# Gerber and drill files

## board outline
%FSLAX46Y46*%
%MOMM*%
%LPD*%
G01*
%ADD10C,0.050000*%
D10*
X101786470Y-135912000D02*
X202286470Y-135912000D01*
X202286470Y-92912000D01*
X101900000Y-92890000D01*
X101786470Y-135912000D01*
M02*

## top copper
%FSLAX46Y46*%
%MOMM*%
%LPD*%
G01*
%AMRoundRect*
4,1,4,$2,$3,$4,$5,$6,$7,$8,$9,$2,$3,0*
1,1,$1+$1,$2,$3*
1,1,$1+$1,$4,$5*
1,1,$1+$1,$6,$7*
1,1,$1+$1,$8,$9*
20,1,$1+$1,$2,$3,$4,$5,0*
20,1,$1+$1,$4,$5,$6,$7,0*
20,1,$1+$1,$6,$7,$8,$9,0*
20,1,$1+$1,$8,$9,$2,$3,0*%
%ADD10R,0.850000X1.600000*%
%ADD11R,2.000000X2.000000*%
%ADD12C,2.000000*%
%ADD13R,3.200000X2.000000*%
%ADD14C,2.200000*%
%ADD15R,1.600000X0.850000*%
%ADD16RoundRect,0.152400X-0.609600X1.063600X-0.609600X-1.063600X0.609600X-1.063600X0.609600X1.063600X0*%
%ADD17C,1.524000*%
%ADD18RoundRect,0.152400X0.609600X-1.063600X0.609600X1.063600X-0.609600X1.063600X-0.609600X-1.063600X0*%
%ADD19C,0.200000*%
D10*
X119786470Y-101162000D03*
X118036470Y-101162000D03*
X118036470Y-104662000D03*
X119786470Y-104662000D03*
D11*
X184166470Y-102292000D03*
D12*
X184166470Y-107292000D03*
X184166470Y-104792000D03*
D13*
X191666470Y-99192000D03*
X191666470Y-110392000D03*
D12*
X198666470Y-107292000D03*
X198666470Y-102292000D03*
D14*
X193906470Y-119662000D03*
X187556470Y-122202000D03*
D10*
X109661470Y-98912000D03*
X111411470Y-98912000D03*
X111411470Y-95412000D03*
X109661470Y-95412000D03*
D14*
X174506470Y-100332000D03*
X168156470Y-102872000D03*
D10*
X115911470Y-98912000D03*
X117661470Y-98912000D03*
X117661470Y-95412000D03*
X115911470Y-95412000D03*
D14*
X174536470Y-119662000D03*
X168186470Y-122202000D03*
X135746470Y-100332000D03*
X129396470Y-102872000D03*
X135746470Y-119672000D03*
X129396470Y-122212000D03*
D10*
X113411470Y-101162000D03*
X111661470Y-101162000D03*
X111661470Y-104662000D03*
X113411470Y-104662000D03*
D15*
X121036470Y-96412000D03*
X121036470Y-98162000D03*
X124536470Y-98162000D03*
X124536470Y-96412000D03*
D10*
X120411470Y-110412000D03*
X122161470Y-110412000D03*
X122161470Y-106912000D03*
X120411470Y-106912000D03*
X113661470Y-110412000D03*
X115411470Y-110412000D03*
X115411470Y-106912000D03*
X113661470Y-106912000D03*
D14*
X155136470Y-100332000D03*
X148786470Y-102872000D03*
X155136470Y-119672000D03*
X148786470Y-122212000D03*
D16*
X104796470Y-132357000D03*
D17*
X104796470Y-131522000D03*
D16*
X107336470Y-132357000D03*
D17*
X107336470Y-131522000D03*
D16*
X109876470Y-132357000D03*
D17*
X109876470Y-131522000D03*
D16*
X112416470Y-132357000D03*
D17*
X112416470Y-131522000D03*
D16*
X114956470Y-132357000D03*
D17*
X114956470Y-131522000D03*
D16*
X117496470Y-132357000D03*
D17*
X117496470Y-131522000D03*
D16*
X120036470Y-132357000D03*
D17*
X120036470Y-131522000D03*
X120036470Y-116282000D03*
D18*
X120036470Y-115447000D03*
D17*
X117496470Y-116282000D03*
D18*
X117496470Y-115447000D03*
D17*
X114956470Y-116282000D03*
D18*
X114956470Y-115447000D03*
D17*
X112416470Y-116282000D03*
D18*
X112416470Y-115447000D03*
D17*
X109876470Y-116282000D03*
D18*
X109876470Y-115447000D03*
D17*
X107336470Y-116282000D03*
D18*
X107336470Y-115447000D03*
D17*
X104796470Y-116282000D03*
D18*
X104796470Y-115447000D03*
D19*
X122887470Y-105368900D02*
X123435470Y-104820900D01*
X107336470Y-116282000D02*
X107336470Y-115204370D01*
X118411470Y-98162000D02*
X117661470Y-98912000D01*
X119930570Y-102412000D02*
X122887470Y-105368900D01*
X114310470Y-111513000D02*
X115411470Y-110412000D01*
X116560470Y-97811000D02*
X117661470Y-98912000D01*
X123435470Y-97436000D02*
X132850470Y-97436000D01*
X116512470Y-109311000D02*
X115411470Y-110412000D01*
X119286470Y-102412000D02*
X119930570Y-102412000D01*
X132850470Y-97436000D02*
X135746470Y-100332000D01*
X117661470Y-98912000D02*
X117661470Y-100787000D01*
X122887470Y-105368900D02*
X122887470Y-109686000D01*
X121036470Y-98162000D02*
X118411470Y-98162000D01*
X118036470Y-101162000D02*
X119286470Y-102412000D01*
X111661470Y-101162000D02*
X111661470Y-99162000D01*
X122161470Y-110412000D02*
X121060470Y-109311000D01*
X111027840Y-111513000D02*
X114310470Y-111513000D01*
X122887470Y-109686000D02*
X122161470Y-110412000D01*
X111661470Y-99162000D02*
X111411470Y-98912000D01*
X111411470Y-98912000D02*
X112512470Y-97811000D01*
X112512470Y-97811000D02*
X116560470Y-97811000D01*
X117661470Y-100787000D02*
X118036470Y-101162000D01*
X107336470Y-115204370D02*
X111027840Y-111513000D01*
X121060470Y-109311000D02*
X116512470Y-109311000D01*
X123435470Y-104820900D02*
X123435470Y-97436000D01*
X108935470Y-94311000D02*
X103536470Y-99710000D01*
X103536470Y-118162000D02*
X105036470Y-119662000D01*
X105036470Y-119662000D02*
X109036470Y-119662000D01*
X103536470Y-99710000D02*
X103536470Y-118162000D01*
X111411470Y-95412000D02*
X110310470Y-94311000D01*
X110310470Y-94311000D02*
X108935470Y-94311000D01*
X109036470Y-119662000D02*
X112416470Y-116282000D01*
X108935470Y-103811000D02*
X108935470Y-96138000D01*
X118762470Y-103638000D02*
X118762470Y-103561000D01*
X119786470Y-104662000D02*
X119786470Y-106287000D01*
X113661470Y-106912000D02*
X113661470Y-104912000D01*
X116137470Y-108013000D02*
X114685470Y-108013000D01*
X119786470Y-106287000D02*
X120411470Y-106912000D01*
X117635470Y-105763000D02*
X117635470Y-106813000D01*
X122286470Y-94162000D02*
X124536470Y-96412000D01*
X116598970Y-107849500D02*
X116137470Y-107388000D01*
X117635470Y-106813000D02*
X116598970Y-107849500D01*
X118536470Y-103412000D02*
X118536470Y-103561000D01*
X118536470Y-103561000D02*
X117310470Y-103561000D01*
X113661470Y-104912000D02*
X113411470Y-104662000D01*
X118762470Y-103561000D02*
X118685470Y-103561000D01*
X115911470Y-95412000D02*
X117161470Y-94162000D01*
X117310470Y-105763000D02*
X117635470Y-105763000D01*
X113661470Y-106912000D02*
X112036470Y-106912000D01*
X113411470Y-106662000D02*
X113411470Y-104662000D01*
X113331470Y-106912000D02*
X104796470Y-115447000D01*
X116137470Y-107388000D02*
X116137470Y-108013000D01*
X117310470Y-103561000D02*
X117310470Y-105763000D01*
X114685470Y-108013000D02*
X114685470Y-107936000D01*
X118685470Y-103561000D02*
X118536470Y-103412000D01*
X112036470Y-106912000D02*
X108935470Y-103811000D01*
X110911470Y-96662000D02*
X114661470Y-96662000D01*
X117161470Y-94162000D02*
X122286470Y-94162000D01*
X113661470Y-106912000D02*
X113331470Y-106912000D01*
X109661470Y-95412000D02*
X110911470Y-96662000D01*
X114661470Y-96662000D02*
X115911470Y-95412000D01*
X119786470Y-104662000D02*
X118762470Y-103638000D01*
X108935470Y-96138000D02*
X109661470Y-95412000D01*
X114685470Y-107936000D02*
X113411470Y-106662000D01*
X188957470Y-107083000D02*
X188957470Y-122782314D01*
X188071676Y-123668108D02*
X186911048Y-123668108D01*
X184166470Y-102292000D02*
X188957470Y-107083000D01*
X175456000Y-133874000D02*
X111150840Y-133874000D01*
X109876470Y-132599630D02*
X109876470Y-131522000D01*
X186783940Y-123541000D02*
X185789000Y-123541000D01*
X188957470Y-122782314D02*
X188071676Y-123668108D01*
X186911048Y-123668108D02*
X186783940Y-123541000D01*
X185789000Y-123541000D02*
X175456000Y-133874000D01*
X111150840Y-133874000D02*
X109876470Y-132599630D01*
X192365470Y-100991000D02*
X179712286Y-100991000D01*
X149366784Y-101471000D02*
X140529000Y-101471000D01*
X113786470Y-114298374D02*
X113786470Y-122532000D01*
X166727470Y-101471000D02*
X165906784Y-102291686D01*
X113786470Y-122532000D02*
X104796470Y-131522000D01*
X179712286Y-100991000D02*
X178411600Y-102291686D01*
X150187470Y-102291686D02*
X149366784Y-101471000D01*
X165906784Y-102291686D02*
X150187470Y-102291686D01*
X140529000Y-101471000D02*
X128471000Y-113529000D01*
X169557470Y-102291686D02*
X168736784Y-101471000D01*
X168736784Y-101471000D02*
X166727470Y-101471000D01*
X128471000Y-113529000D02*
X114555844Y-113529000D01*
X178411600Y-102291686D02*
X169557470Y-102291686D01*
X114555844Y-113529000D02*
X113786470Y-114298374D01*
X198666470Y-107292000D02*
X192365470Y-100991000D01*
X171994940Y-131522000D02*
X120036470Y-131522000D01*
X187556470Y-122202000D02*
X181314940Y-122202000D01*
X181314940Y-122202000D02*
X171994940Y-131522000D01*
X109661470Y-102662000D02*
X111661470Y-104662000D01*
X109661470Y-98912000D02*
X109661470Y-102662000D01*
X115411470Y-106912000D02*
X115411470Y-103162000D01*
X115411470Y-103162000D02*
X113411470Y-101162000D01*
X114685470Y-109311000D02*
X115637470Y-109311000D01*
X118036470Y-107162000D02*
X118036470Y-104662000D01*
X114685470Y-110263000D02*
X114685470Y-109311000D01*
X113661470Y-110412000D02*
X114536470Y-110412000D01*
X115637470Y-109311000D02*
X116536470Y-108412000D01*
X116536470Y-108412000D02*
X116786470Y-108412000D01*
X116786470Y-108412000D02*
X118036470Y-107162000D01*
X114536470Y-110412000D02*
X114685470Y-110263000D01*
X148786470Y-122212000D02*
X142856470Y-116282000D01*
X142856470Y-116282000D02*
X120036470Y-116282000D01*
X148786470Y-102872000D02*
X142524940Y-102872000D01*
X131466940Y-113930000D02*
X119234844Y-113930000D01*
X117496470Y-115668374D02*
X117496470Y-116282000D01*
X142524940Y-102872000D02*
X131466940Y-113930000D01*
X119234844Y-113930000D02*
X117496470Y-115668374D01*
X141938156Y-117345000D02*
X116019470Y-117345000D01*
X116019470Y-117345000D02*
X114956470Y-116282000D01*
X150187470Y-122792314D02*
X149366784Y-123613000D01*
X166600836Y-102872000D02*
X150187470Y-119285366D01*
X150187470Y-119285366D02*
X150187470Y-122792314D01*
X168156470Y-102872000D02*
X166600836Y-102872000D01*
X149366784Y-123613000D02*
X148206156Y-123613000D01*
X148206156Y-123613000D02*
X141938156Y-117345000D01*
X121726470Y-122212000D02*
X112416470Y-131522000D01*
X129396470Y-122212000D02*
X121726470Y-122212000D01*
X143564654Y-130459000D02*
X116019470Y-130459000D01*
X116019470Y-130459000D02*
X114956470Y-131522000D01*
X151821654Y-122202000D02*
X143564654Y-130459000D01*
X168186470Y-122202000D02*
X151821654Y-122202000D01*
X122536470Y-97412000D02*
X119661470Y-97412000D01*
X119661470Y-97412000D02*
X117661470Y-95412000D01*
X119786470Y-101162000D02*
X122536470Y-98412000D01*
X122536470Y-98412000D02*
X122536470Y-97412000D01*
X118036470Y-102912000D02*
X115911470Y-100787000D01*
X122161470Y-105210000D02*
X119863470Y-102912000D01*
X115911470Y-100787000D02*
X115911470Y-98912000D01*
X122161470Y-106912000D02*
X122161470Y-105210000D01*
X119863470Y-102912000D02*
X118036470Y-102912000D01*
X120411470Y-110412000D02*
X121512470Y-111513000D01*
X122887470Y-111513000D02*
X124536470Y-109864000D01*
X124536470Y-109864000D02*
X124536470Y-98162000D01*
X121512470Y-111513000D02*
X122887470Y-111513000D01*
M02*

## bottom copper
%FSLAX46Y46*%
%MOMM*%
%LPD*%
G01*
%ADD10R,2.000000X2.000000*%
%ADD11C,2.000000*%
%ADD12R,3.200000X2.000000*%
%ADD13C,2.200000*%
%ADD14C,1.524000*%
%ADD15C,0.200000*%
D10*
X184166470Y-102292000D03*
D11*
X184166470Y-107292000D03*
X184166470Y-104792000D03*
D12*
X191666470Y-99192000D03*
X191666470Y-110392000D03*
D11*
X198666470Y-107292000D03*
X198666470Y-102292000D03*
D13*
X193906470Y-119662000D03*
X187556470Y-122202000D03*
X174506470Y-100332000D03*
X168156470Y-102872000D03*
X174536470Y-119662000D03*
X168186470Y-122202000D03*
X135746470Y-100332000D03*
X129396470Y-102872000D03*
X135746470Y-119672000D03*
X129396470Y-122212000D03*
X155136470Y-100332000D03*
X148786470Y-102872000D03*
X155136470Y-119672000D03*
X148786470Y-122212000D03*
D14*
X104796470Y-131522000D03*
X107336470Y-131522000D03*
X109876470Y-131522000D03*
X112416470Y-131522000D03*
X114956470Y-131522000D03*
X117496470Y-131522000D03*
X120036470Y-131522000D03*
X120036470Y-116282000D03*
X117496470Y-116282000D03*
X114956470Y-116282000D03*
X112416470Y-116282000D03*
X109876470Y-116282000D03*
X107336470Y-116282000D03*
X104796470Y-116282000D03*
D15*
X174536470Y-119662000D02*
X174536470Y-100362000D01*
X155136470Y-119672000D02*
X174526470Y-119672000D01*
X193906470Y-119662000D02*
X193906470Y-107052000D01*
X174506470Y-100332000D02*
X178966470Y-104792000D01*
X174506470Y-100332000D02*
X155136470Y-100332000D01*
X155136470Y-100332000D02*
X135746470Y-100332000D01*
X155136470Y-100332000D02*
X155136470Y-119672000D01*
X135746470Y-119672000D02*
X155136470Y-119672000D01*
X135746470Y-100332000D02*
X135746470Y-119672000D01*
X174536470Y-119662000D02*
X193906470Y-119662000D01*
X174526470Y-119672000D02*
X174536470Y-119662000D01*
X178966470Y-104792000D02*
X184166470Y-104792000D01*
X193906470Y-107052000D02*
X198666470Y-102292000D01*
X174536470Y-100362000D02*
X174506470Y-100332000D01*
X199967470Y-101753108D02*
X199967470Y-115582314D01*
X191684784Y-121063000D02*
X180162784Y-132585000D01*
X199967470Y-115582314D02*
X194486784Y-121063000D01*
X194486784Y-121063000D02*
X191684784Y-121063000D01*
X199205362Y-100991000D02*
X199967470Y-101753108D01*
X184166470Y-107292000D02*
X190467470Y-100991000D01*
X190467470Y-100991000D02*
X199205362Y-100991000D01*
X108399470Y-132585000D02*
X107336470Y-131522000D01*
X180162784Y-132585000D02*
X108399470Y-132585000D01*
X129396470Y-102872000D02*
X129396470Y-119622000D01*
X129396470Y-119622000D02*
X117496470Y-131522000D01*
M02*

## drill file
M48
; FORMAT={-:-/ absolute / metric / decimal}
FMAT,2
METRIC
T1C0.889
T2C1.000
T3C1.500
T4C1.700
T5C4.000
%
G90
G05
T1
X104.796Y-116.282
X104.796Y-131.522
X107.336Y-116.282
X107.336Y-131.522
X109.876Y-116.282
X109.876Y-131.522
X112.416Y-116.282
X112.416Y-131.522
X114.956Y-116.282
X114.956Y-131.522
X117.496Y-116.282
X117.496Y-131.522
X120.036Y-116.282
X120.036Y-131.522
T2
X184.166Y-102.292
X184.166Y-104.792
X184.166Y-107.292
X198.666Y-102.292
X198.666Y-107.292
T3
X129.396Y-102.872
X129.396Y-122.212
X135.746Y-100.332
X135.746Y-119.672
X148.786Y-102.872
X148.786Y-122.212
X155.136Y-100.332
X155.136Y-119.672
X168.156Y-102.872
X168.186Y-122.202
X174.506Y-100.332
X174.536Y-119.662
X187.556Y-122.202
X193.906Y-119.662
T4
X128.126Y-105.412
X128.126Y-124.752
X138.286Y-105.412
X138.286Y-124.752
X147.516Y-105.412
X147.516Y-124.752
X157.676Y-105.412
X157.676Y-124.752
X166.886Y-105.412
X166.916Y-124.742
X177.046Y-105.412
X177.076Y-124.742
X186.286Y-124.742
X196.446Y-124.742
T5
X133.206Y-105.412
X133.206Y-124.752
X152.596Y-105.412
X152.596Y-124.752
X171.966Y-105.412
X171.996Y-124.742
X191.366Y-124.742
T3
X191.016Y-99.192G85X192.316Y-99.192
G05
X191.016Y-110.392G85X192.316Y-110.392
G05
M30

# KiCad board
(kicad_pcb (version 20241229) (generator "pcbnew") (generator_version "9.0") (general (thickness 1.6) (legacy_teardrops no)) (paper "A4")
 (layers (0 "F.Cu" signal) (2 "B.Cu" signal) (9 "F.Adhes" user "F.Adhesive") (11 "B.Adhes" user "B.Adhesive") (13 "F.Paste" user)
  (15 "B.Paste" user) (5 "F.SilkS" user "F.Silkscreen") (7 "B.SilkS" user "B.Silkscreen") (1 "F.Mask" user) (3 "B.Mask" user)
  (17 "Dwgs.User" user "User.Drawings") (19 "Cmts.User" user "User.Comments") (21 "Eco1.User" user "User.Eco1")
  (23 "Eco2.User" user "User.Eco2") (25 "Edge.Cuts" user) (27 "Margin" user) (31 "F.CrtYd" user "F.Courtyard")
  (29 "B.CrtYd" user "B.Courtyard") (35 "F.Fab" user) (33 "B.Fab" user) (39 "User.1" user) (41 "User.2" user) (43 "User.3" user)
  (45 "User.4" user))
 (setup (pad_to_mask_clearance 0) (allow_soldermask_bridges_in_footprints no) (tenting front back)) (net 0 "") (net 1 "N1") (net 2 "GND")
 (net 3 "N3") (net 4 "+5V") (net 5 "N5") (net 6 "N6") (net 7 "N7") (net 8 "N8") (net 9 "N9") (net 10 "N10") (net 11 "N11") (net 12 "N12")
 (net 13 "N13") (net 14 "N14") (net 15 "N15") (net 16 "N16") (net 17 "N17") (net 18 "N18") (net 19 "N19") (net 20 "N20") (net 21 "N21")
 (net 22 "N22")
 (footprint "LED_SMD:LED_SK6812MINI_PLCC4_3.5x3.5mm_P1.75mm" (layer "F.Cu") (at 118.91147 102.912 -90)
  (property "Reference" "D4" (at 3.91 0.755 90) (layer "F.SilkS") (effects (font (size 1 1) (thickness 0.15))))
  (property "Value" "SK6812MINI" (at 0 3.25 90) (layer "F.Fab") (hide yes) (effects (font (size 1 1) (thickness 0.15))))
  (pad "1" smd rect (at -1.75 -0.875 270) (size 1.6 0.85) (layers "F.Cu" "F.Mask" "F.Paste") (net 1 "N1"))
  (pad "2" smd rect (at -1.75 0.875 270) (size 1.6 0.85) (layers "F.Cu" "F.Mask" "F.Paste") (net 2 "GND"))
  (pad "3" smd rect (at 1.75 0.875 270) (size 1.6 0.85) (layers "F.Cu" "F.Mask" "F.Paste") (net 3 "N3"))
  (pad "4" smd rect (at 1.75 -0.875 270) (size 1.6 0.85) (layers "F.Cu" "F.Mask" "F.Paste") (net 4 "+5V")))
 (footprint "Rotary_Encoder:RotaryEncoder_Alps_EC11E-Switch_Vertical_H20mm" (layer "F.Cu") (at 184.16647 102.292)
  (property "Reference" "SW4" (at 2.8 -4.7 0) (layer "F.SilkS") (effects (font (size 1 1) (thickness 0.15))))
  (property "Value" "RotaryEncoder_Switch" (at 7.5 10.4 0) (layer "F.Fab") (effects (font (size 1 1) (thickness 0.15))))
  (pad "A" thru_hole rect (at 0 0) (size 2 2) (drill 1) (layers "*.Cu" "*.Mask") (remove_unused_layers no) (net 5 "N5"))
  (pad "B" thru_hole circle (at 0 5) (size 2 2) (drill 1) (layers "*.Cu" "*.Mask") (remove_unused_layers no) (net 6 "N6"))
  (pad "C" thru_hole circle (at 0 2.5) (size 2 2) (drill 1) (layers "*.Cu" "*.Mask") (remove_unused_layers no) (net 2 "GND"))
  (pad "MP" thru_hole rect (at 7.5 -3.1) (size 3.2 2) (drill oval 2.8 1.5) (layers "*.Cu" "*.Mask") (remove_unused_layers no))
  (pad "MP" thru_hole rect (at 7.5 8.1) (size 3.2 2) (drill oval 2.8 1.5) (layers "*.Cu" "*.Mask") (remove_unused_layers no))
  (pad "S1" thru_hole circle (at 14.5 5) (size 2 2) (drill 1) (layers "*.Cu" "*.Mask") (remove_unused_layers no) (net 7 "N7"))
  (pad "S2" thru_hole circle (at 14.5 0) (size 2 2) (drill 1) (layers "*.Cu" "*.Mask") (remove_unused_layers no) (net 2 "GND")))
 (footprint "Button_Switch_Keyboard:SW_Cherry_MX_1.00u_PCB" (layer "F.Cu") (at 193.90647 119.662)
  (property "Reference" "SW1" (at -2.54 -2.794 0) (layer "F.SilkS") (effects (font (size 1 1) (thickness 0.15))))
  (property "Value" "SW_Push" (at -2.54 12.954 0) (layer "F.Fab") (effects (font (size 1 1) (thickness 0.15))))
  (pad "" np_thru_hole circle (at -7.62 5.08) (size 1.7 1.7) (drill 1.7) (layers "*.Cu" "*.Mask"))
  (pad "" np_thru_hole circle (at -2.54 5.08) (size 4 4) (drill 4) (layers "*.Cu" "*.Mask"))
  (pad "" np_thru_hole circle (at 2.54 5.08) (size 1.7 1.7) (drill 1.7) (layers "*.Cu" "*.Mask"))
  (pad "1" thru_hole circle (at 0 0) (size 2.2 2.2) (drill 1.5) (layers "*.Cu" "*.Mask") (remove_unused_layers no) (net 2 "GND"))
  (pad "2" thru_hole circle (at -6.35 2.54) (size 2.2 2.2) (drill 1.5) (layers "*.Cu" "*.Mask") (remove_unused_layers no) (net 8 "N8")))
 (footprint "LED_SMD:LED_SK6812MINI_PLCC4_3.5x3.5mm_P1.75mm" (layer "F.Cu") (at 110.53647 97.162 90)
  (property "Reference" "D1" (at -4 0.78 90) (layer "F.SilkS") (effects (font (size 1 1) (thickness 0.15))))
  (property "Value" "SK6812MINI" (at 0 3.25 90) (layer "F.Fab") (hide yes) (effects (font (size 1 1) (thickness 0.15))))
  (pad "1" smd rect (at -1.75 -0.875 90) (size 1.6 0.85) (layers "F.Cu" "F.Mask" "F.Paste") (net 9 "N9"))
  (pad "2" smd rect (at -1.75 0.875 90) (size 1.6 0.85) (layers "F.Cu" "F.Mask" "F.Paste") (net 2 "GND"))
  (pad "3" smd rect (at 1.75 0.875 90) (size 1.6 0.85) (layers "F.Cu" "F.Mask" "F.Paste") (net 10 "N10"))
  (pad "4" smd rect (at 1.75 -0.875 90) (size 1.6 0.85) (layers "F.Cu" "F.Mask" "F.Paste") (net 4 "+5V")))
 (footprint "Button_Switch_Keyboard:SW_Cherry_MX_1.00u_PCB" (layer "F.Cu") (at 174.50647 100.332)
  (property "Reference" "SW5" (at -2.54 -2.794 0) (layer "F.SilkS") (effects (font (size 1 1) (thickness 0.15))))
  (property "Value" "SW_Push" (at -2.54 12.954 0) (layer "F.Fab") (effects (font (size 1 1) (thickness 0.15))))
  (pad "" np_thru_hole circle (at -7.62 5.08) (size 1.7 1.7) (drill 1.7) (layers "*.Cu" "*.Mask"))
  (pad "" np_thru_hole circle (at -2.54 5.08) (size 4 4) (drill 4) (layers "*.Cu" "*.Mask"))
  (pad "" np_thru_hole circle (at 2.54 5.08) (size 1.7 1.7) (drill 1.7) (layers "*.Cu" "*.Mask"))
  (pad "1" thru_hole circle (at 0 0) (size 2.2 2.2) (drill 1.5) (layers "*.Cu" "*.Mask") (remove_unused_layers no) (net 2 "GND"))
  (pad "2" thru_hole circle (at -6.35 2.54) (size 2.2 2.2) (drill 1.5) (layers "*.Cu" "*.Mask") (remove_unused_layers no) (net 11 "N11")))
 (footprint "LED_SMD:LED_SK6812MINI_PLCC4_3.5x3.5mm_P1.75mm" (layer "F.Cu") (at 116.78647 97.162 90)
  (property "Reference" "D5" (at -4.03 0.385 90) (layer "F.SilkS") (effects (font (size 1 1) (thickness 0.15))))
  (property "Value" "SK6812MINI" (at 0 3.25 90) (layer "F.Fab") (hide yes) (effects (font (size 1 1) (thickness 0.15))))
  (pad "1" smd rect (at -1.75 -0.875 90) (size 1.6 0.85) (layers "F.Cu" "F.Mask" "F.Paste") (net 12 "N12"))
  (pad "2" smd rect (at -1.75 0.875 90) (size 1.6 0.85) (layers "F.Cu" "F.Mask" "F.Paste") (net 2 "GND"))
  (pad "3" smd rect (at 1.75 0.875 90) (size 1.6 0.85) (layers "F.Cu" "F.Mask" "F.Paste") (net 1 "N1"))
  (pad "4" smd rect (at 1.75 -0.875 90) (size 1.6 0.85) (layers "F.Cu" "F.Mask" "F.Paste") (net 4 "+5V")))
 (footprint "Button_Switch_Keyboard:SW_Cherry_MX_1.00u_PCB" (layer "F.Cu") (at 174.53647 119.662)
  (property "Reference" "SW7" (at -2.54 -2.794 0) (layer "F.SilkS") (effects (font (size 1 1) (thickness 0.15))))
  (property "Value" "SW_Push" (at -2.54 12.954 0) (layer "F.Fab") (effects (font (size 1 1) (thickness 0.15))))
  (pad "" np_thru_hole circle (at -7.62 5.08) (size 1.7 1.7) (drill 1.7) (layers "*.Cu" "*.Mask"))
  (pad "" np_thru_hole circle (at -2.54 5.08) (size 4 4) (drill 4) (layers "*.Cu" "*.Mask"))
  (pad "" np_thru_hole circle (at 2.54 5.08) (size 1.7 1.7) (drill 1.7) (layers "*.Cu" "*.Mask"))
  (pad "1" thru_hole circle (at 0 0) (size 2.2 2.2) (drill 1.5) (layers "*.Cu" "*.Mask") (remove_unused_layers no) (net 2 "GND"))
  (pad "2" thru_hole circle (at -6.35 2.54) (size 2.2 2.2) (drill 1.5) (layers "*.Cu" "*.Mask") (remove_unused_layers no) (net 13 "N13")))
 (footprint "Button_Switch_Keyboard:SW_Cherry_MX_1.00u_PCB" (layer "F.Cu") (at 135.74647 100.332)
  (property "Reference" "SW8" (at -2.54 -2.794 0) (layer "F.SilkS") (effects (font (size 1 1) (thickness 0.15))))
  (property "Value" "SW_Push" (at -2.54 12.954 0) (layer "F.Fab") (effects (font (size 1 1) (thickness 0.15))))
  (pad "" np_thru_hole circle (at -7.62 5.08) (size 1.7 1.7) (drill 1.7) (layers "*.Cu" "*.Mask"))
  (pad "" np_thru_hole circle (at -2.54 5.08) (size 4 4) (drill 4) (layers "*.Cu" "*.Mask"))
  (pad "" np_thru_hole circle (at 2.54 5.08) (size 1.7 1.7) (drill 1.7) (layers "*.Cu" "*.Mask"))
  (pad "1" thru_hole circle (at 0 0) (size 2.2 2.2) (drill 1.5) (layers "*.Cu" "*.Mask") (remove_unused_layers no) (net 2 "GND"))
  (pad "2" thru_hole circle (at -6.35 2.54) (size 2.2 2.2) (drill 1.5) (layers "*.Cu" "*.Mask") (remove_unused_layers no) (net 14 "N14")))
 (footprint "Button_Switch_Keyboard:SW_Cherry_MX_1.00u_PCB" (layer "F.Cu") (at 135.74647 119.672)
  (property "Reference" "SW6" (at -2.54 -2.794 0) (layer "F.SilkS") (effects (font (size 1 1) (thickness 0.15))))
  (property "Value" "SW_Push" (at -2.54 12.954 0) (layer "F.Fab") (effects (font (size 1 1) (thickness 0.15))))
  (pad "" np_thru_hole circle (at -7.62 5.08) (size 1.7 1.7) (drill 1.7) (layers "*.Cu" "*.Mask"))
  (pad "" np_thru_hole circle (at -2.54 5.08) (size 4 4) (drill 4) (layers "*.Cu" "*.Mask"))
  (pad "" np_thru_hole circle (at 2.54 5.08) (size 1.7 1.7) (drill 1.7) (layers "*.Cu" "*.Mask"))
  (pad "1" thru_hole circle (at 0 0) (size 2.2 2.2) (drill 1.5) (layers "*.Cu" "*.Mask") (remove_unused_layers no) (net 2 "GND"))
  (pad "2" thru_hole circle (at -6.35 2.54) (size 2.2 2.2) (drill 1.5) (layers "*.Cu" "*.Mask") (remove_unused_layers no) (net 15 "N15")))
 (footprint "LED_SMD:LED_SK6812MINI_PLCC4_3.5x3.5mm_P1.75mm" (layer "F.Cu") (at 112.53647 102.912 -90)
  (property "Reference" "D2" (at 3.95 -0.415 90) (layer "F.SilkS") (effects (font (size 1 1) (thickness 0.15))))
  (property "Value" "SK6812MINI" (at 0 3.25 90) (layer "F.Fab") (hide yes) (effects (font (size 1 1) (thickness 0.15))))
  (pad "1" smd rect (at -1.75 -0.875 270) (size 1.6 0.85) (layers "F.Cu" "F.Mask" "F.Paste") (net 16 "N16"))
  (pad "2" smd rect (at -1.75 0.875 270) (size 1.6 0.85) (layers "F.Cu" "F.Mask" "F.Paste") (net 2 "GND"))
  (pad "3" smd rect (at 1.75 0.875 270) (size 1.6 0.85) (layers "F.Cu" "F.Mask" "F.Paste") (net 9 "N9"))
  (pad "4" smd rect (at 1.75 -0.875 270) (size 1.6 0.85) (layers "F.Cu" "F.Mask" "F.Paste") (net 4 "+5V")))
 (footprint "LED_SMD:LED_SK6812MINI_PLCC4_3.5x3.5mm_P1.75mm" (layer "F.Cu") (at 122.78647 97.287)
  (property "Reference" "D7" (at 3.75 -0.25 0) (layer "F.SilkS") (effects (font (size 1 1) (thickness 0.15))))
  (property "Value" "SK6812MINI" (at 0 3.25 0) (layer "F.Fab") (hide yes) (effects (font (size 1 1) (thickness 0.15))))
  (pad "1" smd rect (at -1.75 -0.875) (size 1.6 0.85) (layers "F.Cu" "F.Mask" "F.Paste") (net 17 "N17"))
  (pad "2" smd rect (at -1.75 0.875) (size 1.6 0.85) (layers "F.Cu" "F.Mask" "F.Paste") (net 2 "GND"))
  (pad "3" smd rect (at 1.75 0.875) (size 1.6 0.85) (layers "F.Cu" "F.Mask" "F.Paste") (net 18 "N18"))
  (pad "4" smd rect (at 1.75 -0.875) (size 1.6 0.85) (layers "F.Cu" "F.Mask" "F.Paste") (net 4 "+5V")))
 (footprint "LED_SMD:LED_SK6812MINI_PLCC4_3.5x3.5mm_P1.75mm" (layer "F.Cu") (at 121.28647 108.662 90)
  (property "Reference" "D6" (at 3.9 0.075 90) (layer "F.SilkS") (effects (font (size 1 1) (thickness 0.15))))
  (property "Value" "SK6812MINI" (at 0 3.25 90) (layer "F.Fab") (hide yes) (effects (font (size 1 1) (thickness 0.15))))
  (pad "1" smd rect (at -1.75 -0.875 90) (size 1.6 0.85) (layers "F.Cu" "F.Mask" "F.Paste") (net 18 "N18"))
  (pad "2" smd rect (at -1.75 0.875 90) (size 1.6 0.85) (layers "F.Cu" "F.Mask" "F.Paste") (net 2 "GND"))
  (pad "3" smd rect (at 1.75 0.875 90) (size 1.6 0.85) (layers "F.Cu" "F.Mask" "F.Paste") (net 12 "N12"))
  (pad "4" smd rect (at 1.75 -0.875 90) (size 1.6 0.85) (layers "F.Cu" "F.Mask" "F.Paste") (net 4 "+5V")))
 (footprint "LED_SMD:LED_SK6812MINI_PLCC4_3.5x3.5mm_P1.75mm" (layer "F.Cu") (at 114.53647 108.662 90)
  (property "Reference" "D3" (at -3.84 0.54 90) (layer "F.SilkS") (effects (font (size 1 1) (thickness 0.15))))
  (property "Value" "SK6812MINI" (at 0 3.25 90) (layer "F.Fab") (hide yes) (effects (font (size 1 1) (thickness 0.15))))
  (pad "1" smd rect (at -1.75 -0.875 90) (size 1.6 0.85) (layers "F.Cu" "F.Mask" "F.Paste") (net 3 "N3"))
  (pad "2" smd rect (at -1.75 0.875 90) (size 1.6 0.85) (layers "F.Cu" "F.Mask" "F.Paste") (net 2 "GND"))
  (pad "3" smd rect (at 1.75 0.875 90) (size 1.6 0.85) (layers "F.Cu" "F.Mask" "F.Paste") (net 16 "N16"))
  (pad "4" smd rect (at 1.75 -0.875 90) (size 1.6 0.85) (layers "F.Cu" "F.Mask" "F.Paste") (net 4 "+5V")))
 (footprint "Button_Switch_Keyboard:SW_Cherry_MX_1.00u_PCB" (layer "F.Cu") (at 155.13647 100.332)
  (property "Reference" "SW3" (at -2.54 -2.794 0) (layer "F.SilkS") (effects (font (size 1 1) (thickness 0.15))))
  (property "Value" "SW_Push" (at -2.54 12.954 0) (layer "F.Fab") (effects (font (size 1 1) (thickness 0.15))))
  (pad "" np_thru_hole circle (at -7.62 5.08) (size 1.7 1.7) (drill 1.7) (layers "*.Cu" "*.Mask"))
  (pad "" np_thru_hole circle (at -2.54 5.08) (size 4 4) (drill 4) (layers "*.Cu" "*.Mask"))
  (pad "" np_thru_hole circle (at 2.54 5.08) (size 1.7 1.7) (drill 1.7) (layers "*.Cu" "*.Mask"))
  (pad "1" thru_hole circle (at 0 0) (size 2.2 2.2) (drill 1.5) (layers "*.Cu" "*.Mask") (remove_unused_layers no) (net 2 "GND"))
  (pad "2" thru_hole circle (at -6.35 2.54) (size 2.2 2.2) (drill 1.5) (layers "*.Cu" "*.Mask") (remove_unused_layers no) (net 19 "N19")))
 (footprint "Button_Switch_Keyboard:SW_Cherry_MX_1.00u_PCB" (layer "F.Cu") (at 155.13647 119.672)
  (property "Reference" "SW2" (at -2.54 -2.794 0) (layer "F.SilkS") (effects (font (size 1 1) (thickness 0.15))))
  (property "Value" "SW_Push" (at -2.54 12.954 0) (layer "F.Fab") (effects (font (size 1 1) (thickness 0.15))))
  (pad "" np_thru_hole circle (at -7.62 5.08) (size 1.7 1.7) (drill 1.7) (layers "*.Cu" "*.Mask"))
  (pad "" np_thru_hole circle (at -2.54 5.08) (size 4 4) (drill 4) (layers "*.Cu" "*.Mask"))
  (pad "" np_thru_hole circle (at 2.54 5.08) (size 1.7 1.7) (drill 1.7) (layers "*.Cu" "*.Mask"))
  (pad "1" thru_hole circle (at 0 0) (size 2.2 2.2) (drill 1.5) (layers "*.Cu" "*.Mask") (remove_unused_layers no) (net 2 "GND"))
  (pad "2" thru_hole circle (at -6.35 2.54) (size 2.2 2.2) (drill 1.5) (layers "*.Cu" "*.Mask") (remove_unused_layers no) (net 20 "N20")))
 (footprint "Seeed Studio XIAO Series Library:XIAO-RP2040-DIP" (layer "F.Cu") (at 112.41647 123.902 90)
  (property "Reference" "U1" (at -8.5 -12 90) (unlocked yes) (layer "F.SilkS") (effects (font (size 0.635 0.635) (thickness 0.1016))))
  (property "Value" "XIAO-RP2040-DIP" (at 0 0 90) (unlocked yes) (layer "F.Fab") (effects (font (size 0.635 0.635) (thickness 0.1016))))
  (pad "1" smd roundrect (at -8.455 -7.62 270) (size 2.432 1.524) (layers "F.Cu" "F.Mask") (roundrect_rratio 0.1) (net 7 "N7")
   (thermal_bridge_angle 45))
  (pad "1" thru_hole circle (at -7.62 -7.62 270) (size 1.524 1.524) (drill 0.889) (layers "*.Cu" "*.Mask") (remove_unused_layers no)
   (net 7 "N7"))
  (pad "2" smd roundrect (at -8.455 -5.08 270) (size 2.432 1.524) (layers "F.Cu" "F.Mask") (roundrect_rratio 0.1) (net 6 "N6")
   (thermal_bridge_angle 45))
  (pad "2" thru_hole circle (at -7.62 -5.08 270) (size 1.524 1.524) (drill 0.889) (layers "*.Cu" "*.Mask") (remove_unused_layers no)
   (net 6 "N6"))
  (pad "3" smd roundrect (at -8.455 -2.54 270) (size 2.432 1.524) (layers "F.Cu" "F.Mask") (roundrect_rratio 0.1) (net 5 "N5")
   (thermal_bridge_angle 45))
  (pad "3" thru_hole circle (at -7.62 -2.54 270) (size 1.524 1.524) (drill 0.889) (layers "*.Cu" "*.Mask") (remove_unused_layers no)
   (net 5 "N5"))
  (pad "4" smd roundrect (at -8.455 0 270) (size 2.432 1.524) (layers "F.Cu" "F.Mask") (roundrect_rratio 0.1) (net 15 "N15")
   (thermal_bridge_angle 45))
  (pad "4" thru_hole circle (at -7.62 0 270) (size 1.524 1.524) (drill 0.889) (layers "*.Cu" "*.Mask") (remove_unused_layers no)
   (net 15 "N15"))
  (pad "5" smd roundrect (at -8.455 2.54 270) (size 2.432 1.524) (layers "F.Cu" "F.Mask") (roundrect_rratio 0.1) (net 13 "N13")
   (thermal_bridge_angle 45))
  (pad "5" thru_hole circle (at -7.62 2.54 270) (size 1.524 1.524) (drill 0.889) (layers "*.Cu" "*.Mask") (remove_unused_layers no)
   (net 13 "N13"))
  (pad "6" smd roundrect (at -8.455 5.08 270) (size 2.432 1.524) (layers "F.Cu" "F.Mask") (roundrect_rratio 0.1) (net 14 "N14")
   (thermal_bridge_angle 45))
  (pad "6" thru_hole circle (at -7.62 5.08 270) (size 1.524 1.524) (drill 0.889) (layers "*.Cu" "*.Mask") (remove_unused_layers no)
   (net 14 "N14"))
  (pad "7" smd roundrect (at -8.455 7.62 270) (size 2.432 1.524) (layers "F.Cu" "F.Mask") (roundrect_rratio 0.1) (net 8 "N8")
   (thermal_bridge_angle 45))
  (pad "7" thru_hole circle (at -7.62 7.62 270) (size 1.524 1.524) (drill 0.889) (layers "*.Cu" "*.Mask") (remove_unused_layers no)
   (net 8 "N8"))
  (pad "8" thru_hole circle (at 7.62 7.62 90) (size 1.524 1.524) (drill 0.889) (layers "*.Cu" "*.Mask") (remove_unused_layers no)
   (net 20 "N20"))
  (pad "8" smd roundrect (at 8.455 7.62 90) (size 2.432 1.524) (layers "F.Cu" "F.Mask") (roundrect_rratio 0.1) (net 20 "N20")
   (thermal_bridge_angle 45))
  (pad "9" thru_hole circle (at 7.62 5.08 90) (size 1.524 1.524) (drill 0.889) (layers "*.Cu" "*.Mask") (remove_unused_layers no)
   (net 19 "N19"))
  (pad "9" smd roundrect (at 8.455 5.08 90) (size 2.432 1.524) (layers "F.Cu" "F.Mask") (roundrect_rratio 0.1) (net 19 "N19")
   (thermal_bridge_angle 45))
  (pad "10" thru_hole circle (at 7.62 2.54 90) (size 1.524 1.524) (drill 0.889) (layers "*.Cu" "*.Mask") (remove_unused_layers no)
   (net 11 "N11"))
  (pad "10" smd roundrect (at 8.455 2.54 90) (size 2.432 1.524) (layers "F.Cu" "F.Mask") (roundrect_rratio 0.1) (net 11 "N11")
   (thermal_bridge_angle 45))
  (pad "11" thru_hole circle (at 7.62 0 90) (size 1.524 1.524) (drill 0.889) (layers "*.Cu" "*.Mask") (remove_unused_layers no)
   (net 10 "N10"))
  (pad "11" smd roundrect (at 8.455 0 90) (size 2.432 1.524) (layers "F.Cu" "F.Mask") (roundrect_rratio 0.1) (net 10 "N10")
   (thermal_bridge_angle 45))
  (pad "12" thru_hole circle (at 7.62 -2.54 90) (size 1.524 1.524) (drill 0.889) (layers "*.Cu" "*.Mask") (remove_unused_layers no)
   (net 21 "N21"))
  (pad "12" smd roundrect (at 8.455 -2.54 90) (size 2.432 1.524) (layers "F.Cu" "F.Mask") (roundrect_rratio 0.1) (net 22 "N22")
   (thermal_bridge_angle 45))
  (pad "13" thru_hole circle (at 7.62 -5.08 90) (size 1.524 1.524) (drill 0.889) (layers "*.Cu" "*.Mask") (remove_unused_layers no)
   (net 2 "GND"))
  (pad "13" smd roundrect (at 8.455 -5.08 90) (size 2.432 1.524) (layers "F.Cu" "F.Mask") (roundrect_rratio 0.1) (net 2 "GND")
   (thermal_bridge_angle 45))
  (pad "14" thru_hole circle (at 7.62 -7.62 90) (size 1.524 1.524) (drill 0.889) (layers "*.Cu" "*.Mask") (remove_unused_layers no)
   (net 4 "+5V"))
  (pad "14" smd roundrect (at 8.455 -7.62 90) (size 2.432 1.524) (layers "F.Cu" "F.Mask") (roundrect_rratio 0.1) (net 4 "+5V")
   (thermal_bridge_angle 45)))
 (gr_poly
  (pts (xy 101.78647 135.912) (xy 202.28647 135.912) (xy 202.28647 92.912) (xy 101.9 92.89)) (stroke (width 0.05) (type solid)) (fill no)
  (layer "Edge.Cuts"))
 (segment (start 122.88747 105.3689) (end 123.43547 104.8209) (width 0.2) (layer "F.Cu") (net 2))
 (segment (start 107.33647 116.282) (end 107.33647 115.20437) (width 0.2) (layer "F.Cu") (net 2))
 (segment (start 118.41147 98.162) (end 117.66147 98.912) (width 0.2) (layer "F.Cu") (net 2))
 (segment (start 119.93057 102.412) (end 122.88747 105.3689) (width 0.2) (layer "F.Cu") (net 2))
 (segment (start 114.31047 111.513) (end 115.41147 110.412) (width 0.2) (layer "F.Cu") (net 2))
 (segment (start 116.56047 97.811) (end 117.66147 98.912) (width 0.2) (layer "F.Cu") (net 2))
 (segment (start 123.43547 97.436) (end 132.85047 97.436) (width 0.2) (layer "F.Cu") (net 2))
 (segment (start 116.51247 109.311) (end 115.41147 110.412) (width 0.2) (layer "F.Cu") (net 2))
 (segment (start 119.28647 102.412) (end 119.93057 102.412) (width 0.2) (layer "F.Cu") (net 2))
 (segment (start 132.85047 97.436) (end 135.74647 100.332) (width 0.2) (layer "F.Cu") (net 2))
 (segment (start 117.66147 98.912) (end 117.66147 100.787) (width 0.2) (layer "F.Cu") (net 2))
 (segment (start 122.88747 105.3689) (end 122.88747 109.686) (width 0.2) (layer "F.Cu") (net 2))
 (segment (start 121.03647 98.162) (end 118.41147 98.162) (width 0.2) (layer "F.Cu") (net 2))
 (segment (start 118.03647 101.162) (end 119.28647 102.412) (width 0.2) (layer "F.Cu") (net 2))
 (segment (start 111.66147 101.162) (end 111.66147 99.162) (width 0.2) (layer "F.Cu") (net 2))
 (segment (start 122.16147 110.412) (end 121.06047 109.311) (width 0.2) (layer "F.Cu") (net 2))
 (segment (start 111.02784 111.513) (end 114.31047 111.513) (width 0.2) (layer "F.Cu") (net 2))
 (segment (start 122.88747 109.686) (end 122.16147 110.412) (width 0.2) (layer "F.Cu") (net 2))
 (segment (start 111.66147 99.162) (end 111.41147 98.912) (width 0.2) (layer "F.Cu") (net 2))
 (segment (start 111.41147 98.912) (end 112.51247 97.811) (width 0.2) (layer "F.Cu") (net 2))
 (segment (start 112.51247 97.811) (end 116.56047 97.811) (width 0.2) (layer "F.Cu") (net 2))
 (segment (start 117.66147 100.787) (end 118.03647 101.162) (width 0.2) (layer "F.Cu") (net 2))
 (segment (start 107.33647 115.20437) (end 111.02784 111.513) (width 0.2) (layer "F.Cu") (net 2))
 (segment (start 121.06047 109.311) (end 116.51247 109.311) (width 0.2) (layer "F.Cu") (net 2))
 (segment (start 123.43547 104.8209) (end 123.43547 97.436) (width 0.2) (layer "F.Cu") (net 2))
 (segment (start 174.53647 119.662) (end 174.53647 100.362) (width 0.2) (layer "B.Cu") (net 2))
 (segment (start 155.13647 119.672) (end 174.52647 119.672) (width 0.2) (layer "B.Cu") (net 2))
 (segment (start 193.90647 119.662) (end 193.90647 107.052) (width 0.2) (layer "B.Cu") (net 2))
 (segment (start 174.50647 100.332) (end 178.96647 104.792) (width 0.2) (layer "B.Cu") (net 2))
 (segment (start 174.50647 100.332) (end 155.13647 100.332) (width 0.2) (layer "B.Cu") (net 2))
 (segment (start 155.13647 100.332) (end 135.74647 100.332) (width 0.2) (layer "B.Cu") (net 2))
 (segment (start 155.13647 100.332) (end 155.13647 119.672) (width 0.2) (layer "B.Cu") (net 2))
 (segment (start 135.74647 119.672) (end 155.13647 119.672) (width 0.2) (layer "B.Cu") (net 2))
 (segment (start 135.74647 100.332) (end 135.74647 119.672) (width 0.2) (layer "B.Cu") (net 2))
 (segment (start 174.53647 119.662) (end 193.90647 119.662) (width 0.2) (layer "B.Cu") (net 2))
 (segment (start 174.52647 119.672) (end 174.53647 119.662) (width 0.2) (layer "B.Cu") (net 2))
 (segment (start 178.96647 104.792) (end 184.16647 104.792) (width 0.2) (layer "B.Cu") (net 2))
 (segment (start 193.90647 107.052) (end 198.66647 102.292) (width 0.2) (layer "B.Cu") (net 2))
 (segment (start 174.53647 100.362) (end 174.50647 100.332) (width 0.2) (layer "B.Cu") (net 2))
 (segment (start 108.93547 94.311) (end 103.53647 99.71) (width 0.2) (layer "F.Cu") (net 10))
 (segment (start 103.53647 118.162) (end 105.03647 119.662) (width 0.2) (layer "F.Cu") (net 10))
 (segment (start 105.03647 119.662) (end 109.03647 119.662) (width 0.2) (layer "F.Cu") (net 10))
 (segment (start 103.53647 99.71) (end 103.53647 118.162) (width 0.2) (layer "F.Cu") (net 10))
 (segment (start 111.41147 95.412) (end 110.31047 94.311) (width 0.2) (layer "F.Cu") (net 10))
 (segment (start 110.31047 94.311) (end 108.93547 94.311) (width 0.2) (layer "F.Cu") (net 10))
 (segment (start 109.03647 119.662) (end 112.41647 116.282) (width 0.2) (layer "F.Cu") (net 10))
 (segment (start 108.93547 103.811) (end 108.93547 96.138) (width 0.2) (layer "F.Cu") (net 4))
 (segment (start 118.76247 103.638) (end 118.76247 103.561) (width 0.2) (layer "F.Cu") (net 4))
 (segment (start 119.78647 104.662) (end 119.78647 106.287) (width 0.2) (layer "F.Cu") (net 4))
 (segment (start 113.66147 106.912) (end 113.66147 104.912) (width 0.2) (layer "F.Cu") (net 4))
 (segment (start 116.13747 108.013) (end 114.68547 108.013) (width 0.2) (layer "F.Cu") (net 4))
 (segment (start 119.78647 106.287) (end 120.41147 106.912) (width 0.2) (layer "F.Cu") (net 4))
 (segment (start 117.63547 105.763) (end 117.63547 106.813) (width 0.2) (layer "F.Cu") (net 4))
 (segment (start 122.28647 94.162) (end 124.53647 96.412) (width 0.2) (layer "F.Cu") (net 4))
 (segment (start 116.59897 107.8495) (end 116.13747 107.388) (width 0.2) (layer "F.Cu") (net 4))
 (segment (start 117.63547 106.813) (end 116.59897 107.8495) (width 0.2) (layer "F.Cu") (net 4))
 (segment (start 118.53647 103.412) (end 118.53647 103.561) (width 0.2) (layer "F.Cu") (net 4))
 (segment (start 118.53647 103.561) (end 117.31047 103.561) (width 0.2) (layer "F.Cu") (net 4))
 (segment (start 113.66147 104.912) (end 113.41147 104.662) (width 0.2) (layer "F.Cu") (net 4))
 (segment (start 118.76247 103.561) (end 118.68547 103.561) (width 0.2) (layer "F.Cu") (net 4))
 (segment (start 115.91147 95.412) (end 117.16147 94.162) (width 0.2) (layer "F.Cu") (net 4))
 (segment (start 117.31047 105.763) (end 117.63547 105.763) (width 0.2) (layer "F.Cu") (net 4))
 (segment (start 113.66147 106.912) (end 112.03647 106.912) (width 0.2) (layer "F.Cu") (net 4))
 (segment (start 113.41147 106.662) (end 113.41147 104.662) (width 0.2) (layer "F.Cu") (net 4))
 (segment (start 113.33147 106.912) (end 104.79647 115.447) (width 0.2) (layer "F.Cu") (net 4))
 (segment (start 116.13747 107.388) (end 116.13747 108.013) (width 0.2) (layer "F.Cu") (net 4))
 (segment (start 117.31047 103.561) (end 117.31047 105.763) (width 0.2) (layer "F.Cu") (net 4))
 (segment (start 114.68547 108.013) (end 114.68547 107.936) (width 0.2) (layer "F.Cu") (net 4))
 (segment (start 118.68547 103.561) (end 118.53647 103.412) (width 0.2) (layer "F.Cu") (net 4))
 (segment (start 112.03647 106.912) (end 108.93547 103.811) (width 0.2) (layer "F.Cu") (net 4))
 (segment (start 110.91147 96.662) (end 114.66147 96.662) (width 0.2) (layer "F.Cu") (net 4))
 (segment (start 117.16147 94.162) (end 122.28647 94.162) (width 0.2) (layer "F.Cu") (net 4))
 (segment (start 113.66147 106.912) (end 113.33147 106.912) (width 0.2) (layer "F.Cu") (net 4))
 (segment (start 109.66147 95.412) (end 110.91147 96.662) (width 0.2) (layer "F.Cu") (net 4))
 (segment (start 114.66147 96.662) (end 115.91147 95.412) (width 0.2) (layer "F.Cu") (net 4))
 (segment (start 119.78647 104.662) (end 118.76247 103.638) (width 0.2) (layer "F.Cu") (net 4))
 (segment (start 108.93547 96.138) (end 109.66147 95.412) (width 0.2) (layer "F.Cu") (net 4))
 (segment (start 114.68547 107.936) (end 113.41147 106.662) (width 0.2) (layer "F.Cu") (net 4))
 (segment (start 199.96747 101.753108) (end 199.96747 115.582314) (width 0.2) (layer "B.Cu") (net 6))
 (segment (start 191.684784 121.063) (end 180.162784 132.585) (width 0.2) (layer "B.Cu") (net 6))
 (segment (start 199.96747 115.582314) (end 194.486784 121.063) (width 0.2) (layer "B.Cu") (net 6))
 (segment (start 194.486784 121.063) (end 191.684784 121.063) (width 0.2) (layer "B.Cu") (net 6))
 (segment (start 199.205362 100.991) (end 199.96747 101.753108) (width 0.2) (layer "B.Cu") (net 6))
 (segment (start 184.16647 107.292) (end 190.46747 100.991) (width 0.2) (layer "B.Cu") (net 6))
 (segment (start 190.46747 100.991) (end 199.205362 100.991) (width 0.2) (layer "B.Cu") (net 6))
 (segment (start 108.39947 132.585) (end 107.33647 131.522) (width 0.2) (layer "B.Cu") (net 6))
 (segment (start 180.162784 132.585) (end 108.39947 132.585) (width 0.2) (layer "B.Cu") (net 6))
 (segment (start 188.95747 107.083) (end 188.95747 122.782314) (width 0.2) (layer "F.Cu") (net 5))
 (segment (start 188.071676 123.668108) (end 186.911048 123.668108) (width 0.2) (layer "F.Cu") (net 5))
 (segment (start 184.16647 102.292) (end 188.95747 107.083) (width 0.2) (layer "F.Cu") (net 5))
 (segment (start 175.456 133.874) (end 111.15084 133.874) (width 0.2) (layer "F.Cu") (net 5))
 (segment (start 109.87647 132.59963) (end 109.87647 131.522) (width 0.2) (layer "F.Cu") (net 5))
 (segment (start 186.78394 123.541) (end 185.789 123.541) (width 0.2) (layer "F.Cu") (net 5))
 (segment (start 188.95747 122.782314) (end 188.071676 123.668108) (width 0.2) (layer "F.Cu") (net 5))
 (segment (start 186.911048 123.668108) (end 186.78394 123.541) (width 0.2) (layer "F.Cu") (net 5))
 (segment (start 185.789 123.541) (end 175.456 133.874) (width 0.2) (layer "F.Cu") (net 5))
 (segment (start 111.15084 133.874) (end 109.87647 132.59963) (width 0.2) (layer "F.Cu") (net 5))
 (segment (start 192.36547 100.991) (end 179.712286 100.991) (width 0.2) (layer "F.Cu") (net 7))
 (segment (start 149.366784 101.471) (end 140.529 101.471) (width 0.2) (layer "F.Cu") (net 7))
 (segment (start 113.78647 114.298374) (end 113.78647 122.532) (width 0.2) (layer "F.Cu") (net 7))
 (segment (start 166.72747 101.471) (end 165.906784 102.291686) (width 0.2) (layer "F.Cu") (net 7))
 (segment (start 113.78647 122.532) (end 104.79647 131.522) (width 0.2) (layer "F.Cu") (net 7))
 (segment (start 179.712286 100.991) (end 178.4116 102.291686) (width 0.2) (layer "F.Cu") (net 7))
 (segment (start 150.18747 102.291686) (end 149.366784 101.471) (width 0.2) (layer "F.Cu") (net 7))
 (segment (start 165.906784 102.291686) (end 150.18747 102.291686) (width 0.2) (layer "F.Cu") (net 7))
 (segment (start 140.529 101.471) (end 128.471 113.529) (width 0.2) (layer "F.Cu") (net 7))
 (segment (start 169.55747 102.291686) (end 168.736784 101.471) (width 0.2) (layer "F.Cu") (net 7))
 (segment (start 168.736784 101.471) (end 166.72747 101.471) (width 0.2) (layer "F.Cu") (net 7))
 (segment (start 128.471 113.529) (end 114.555844 113.529) (width 0.2) (layer "F.Cu") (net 7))
 (segment (start 178.4116 102.291686) (end 169.55747 102.291686) (width 0.2) (layer "F.Cu") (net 7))
 (segment (start 114.555844 113.529) (end 113.78647 114.298374) (width 0.2) (layer "F.Cu") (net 7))
 (segment (start 198.66647 107.292) (end 192.36547 100.991) (width 0.2) (layer "F.Cu") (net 7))
 (segment (start 171.99494 131.522) (end 120.03647 131.522) (width 0.2) (layer "F.Cu") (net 8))
 (segment (start 187.55647 122.202) (end 181.31494 122.202) (width 0.2) (layer "F.Cu") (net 8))
 (segment (start 181.31494 122.202) (end 171.99494 131.522) (width 0.2) (layer "F.Cu") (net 8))
 (segment (start 109.66147 102.662) (end 111.66147 104.662) (width 0.2) (layer "F.Cu") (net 9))
 (segment (start 109.66147 98.912) (end 109.66147 102.662) (width 0.2) (layer "F.Cu") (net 9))
 (segment (start 115.41147 106.912) (end 115.41147 103.162) (width 0.2) (layer "F.Cu") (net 16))
 (segment (start 115.41147 103.162) (end 113.41147 101.162) (width 0.2) (layer "F.Cu") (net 16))
 (segment (start 114.68547 109.311) (end 115.63747 109.311) (width 0.2) (layer "F.Cu") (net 3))
 (segment (start 118.03647 107.162) (end 118.03647 104.662) (width 0.2) (layer "F.Cu") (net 3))
 (segment (start 114.68547 110.263) (end 114.68547 109.311) (width 0.2) (layer "F.Cu") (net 3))
 (segment (start 113.66147 110.412) (end 114.53647 110.412) (width 0.2) (layer "F.Cu") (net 3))
 (segment (start 115.63747 109.311) (end 116.53647 108.412) (width 0.2) (layer "F.Cu") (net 3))
 (segment (start 116.53647 108.412) (end 116.78647 108.412) (width 0.2) (layer "F.Cu") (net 3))
 (segment (start 116.78647 108.412) (end 118.03647 107.162) (width 0.2) (layer "F.Cu") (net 3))
 (segment (start 114.53647 110.412) (end 114.68547 110.263) (width 0.2) (layer "F.Cu") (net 3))
 (segment (start 148.78647 122.212) (end 142.85647 116.282) (width 0.2) (layer "F.Cu") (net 20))
 (segment (start 142.85647 116.282) (end 120.03647 116.282) (width 0.2) (layer "F.Cu") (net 20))
 (segment (start 148.78647 102.872) (end 142.52494 102.872) (width 0.2) (layer "F.Cu") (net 19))
 (segment (start 131.46694 113.93) (end 119.234844 113.93) (width 0.2) (layer "F.Cu") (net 19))
 (segment (start 117.49647 115.668374) (end 117.49647 116.282) (width 0.2) (layer "F.Cu") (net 19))
 (segment (start 142.52494 102.872) (end 131.46694 113.93) (width 0.2) (layer "F.Cu") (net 19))
 (segment (start 119.234844 113.93) (end 117.49647 115.668374) (width 0.2) (layer "F.Cu") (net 19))
 (segment (start 141.938156 117.345) (end 116.01947 117.345) (width 0.2) (layer "F.Cu") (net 11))
 (segment (start 116.01947 117.345) (end 114.95647 116.282) (width 0.2) (layer "F.Cu") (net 11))
 (segment (start 150.18747 122.792314) (end 149.366784 123.613) (width 0.2) (layer "F.Cu") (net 11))
 (segment (start 166.600836 102.872) (end 150.18747 119.285366) (width 0.2) (layer "F.Cu") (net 11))
 (segment (start 150.18747 119.285366) (end 150.18747 122.792314) (width 0.2) (layer "F.Cu") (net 11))
 (segment (start 168.15647 102.872) (end 166.600836 102.872) (width 0.2) (layer "F.Cu") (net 11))
 (segment (start 149.366784 123.613) (end 148.206156 123.613) (width 0.2) (layer "F.Cu") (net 11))
 (segment (start 148.206156 123.613) (end 141.938156 117.345) (width 0.2) (layer "F.Cu") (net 11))
 (segment (start 121.72647 122.212) (end 112.41647 131.522) (width 0.2) (layer "F.Cu") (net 15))
 (segment (start 129.39647 122.212) (end 121.72647 122.212) (width 0.2) (layer "F.Cu") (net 15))
 (segment (start 143.564654 130.459) (end 116.01947 130.459) (width 0.2) (layer "F.Cu") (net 13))
 (segment (start 116.01947 130.459) (end 114.95647 131.522) (width 0.2) (layer "F.Cu") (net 13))
 (segment (start 151.821654 122.202) (end 143.564654 130.459) (width 0.2) (layer "F.Cu") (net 13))
 (segment (start 168.18647 122.202) (end 151.821654 122.202) (width 0.2) (layer "F.Cu") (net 13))
 (segment (start 129.39647 102.872) (end 129.39647 119.622) (width 0.2) (layer "B.Cu") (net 14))
 (segment (start 129.39647 119.622) (end 117.49647 131.522) (width 0.2) (layer "B.Cu") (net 14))
 (segment (start 122.53647 97.412) (end 119.66147 97.412) (width 0.2) (layer "F.Cu") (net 1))
 (segment (start 119.66147 97.412) (end 117.66147 95.412) (width 0.2) (layer "F.Cu") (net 1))
 (segment (start 119.78647 101.162) (end 122.53647 98.412) (width 0.2) (layer "F.Cu") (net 1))
 (segment (start 122.53647 98.412) (end 122.53647 97.412) (width 0.2) (layer "F.Cu") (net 1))
 (segment (start 118.03647 102.912) (end 115.91147 100.787) (width 0.2) (layer "F.Cu") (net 12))
 (segment (start 122.16147 105.21) (end 119.86347 102.912) (width 0.2) (layer "F.Cu") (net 12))
 (segment (start 115.91147 100.787) (end 115.91147 98.912) (width 0.2) (layer "F.Cu") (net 12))
 (segment (start 122.16147 106.912) (end 122.16147 105.21) (width 0.2) (layer "F.Cu") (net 12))
 (segment (start 119.86347 102.912) (end 118.03647 102.912) (width 0.2) (layer "F.Cu") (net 12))
 (segment (start 120.41147 110.412) (end 121.51247 111.513) (width 0.2) (layer "F.Cu") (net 18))
 (segment (start 122.88747 111.513) (end 124.53647 109.864) (width 0.2) (layer "F.Cu") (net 18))
 (segment (start 124.53647 109.864) (end 124.53647 98.162) (width 0.2) (layer "F.Cu") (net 18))
 (segment (start 121.51247 111.513) (end 122.88747 111.513) (width 0.2) (layer "F.Cu") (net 18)))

